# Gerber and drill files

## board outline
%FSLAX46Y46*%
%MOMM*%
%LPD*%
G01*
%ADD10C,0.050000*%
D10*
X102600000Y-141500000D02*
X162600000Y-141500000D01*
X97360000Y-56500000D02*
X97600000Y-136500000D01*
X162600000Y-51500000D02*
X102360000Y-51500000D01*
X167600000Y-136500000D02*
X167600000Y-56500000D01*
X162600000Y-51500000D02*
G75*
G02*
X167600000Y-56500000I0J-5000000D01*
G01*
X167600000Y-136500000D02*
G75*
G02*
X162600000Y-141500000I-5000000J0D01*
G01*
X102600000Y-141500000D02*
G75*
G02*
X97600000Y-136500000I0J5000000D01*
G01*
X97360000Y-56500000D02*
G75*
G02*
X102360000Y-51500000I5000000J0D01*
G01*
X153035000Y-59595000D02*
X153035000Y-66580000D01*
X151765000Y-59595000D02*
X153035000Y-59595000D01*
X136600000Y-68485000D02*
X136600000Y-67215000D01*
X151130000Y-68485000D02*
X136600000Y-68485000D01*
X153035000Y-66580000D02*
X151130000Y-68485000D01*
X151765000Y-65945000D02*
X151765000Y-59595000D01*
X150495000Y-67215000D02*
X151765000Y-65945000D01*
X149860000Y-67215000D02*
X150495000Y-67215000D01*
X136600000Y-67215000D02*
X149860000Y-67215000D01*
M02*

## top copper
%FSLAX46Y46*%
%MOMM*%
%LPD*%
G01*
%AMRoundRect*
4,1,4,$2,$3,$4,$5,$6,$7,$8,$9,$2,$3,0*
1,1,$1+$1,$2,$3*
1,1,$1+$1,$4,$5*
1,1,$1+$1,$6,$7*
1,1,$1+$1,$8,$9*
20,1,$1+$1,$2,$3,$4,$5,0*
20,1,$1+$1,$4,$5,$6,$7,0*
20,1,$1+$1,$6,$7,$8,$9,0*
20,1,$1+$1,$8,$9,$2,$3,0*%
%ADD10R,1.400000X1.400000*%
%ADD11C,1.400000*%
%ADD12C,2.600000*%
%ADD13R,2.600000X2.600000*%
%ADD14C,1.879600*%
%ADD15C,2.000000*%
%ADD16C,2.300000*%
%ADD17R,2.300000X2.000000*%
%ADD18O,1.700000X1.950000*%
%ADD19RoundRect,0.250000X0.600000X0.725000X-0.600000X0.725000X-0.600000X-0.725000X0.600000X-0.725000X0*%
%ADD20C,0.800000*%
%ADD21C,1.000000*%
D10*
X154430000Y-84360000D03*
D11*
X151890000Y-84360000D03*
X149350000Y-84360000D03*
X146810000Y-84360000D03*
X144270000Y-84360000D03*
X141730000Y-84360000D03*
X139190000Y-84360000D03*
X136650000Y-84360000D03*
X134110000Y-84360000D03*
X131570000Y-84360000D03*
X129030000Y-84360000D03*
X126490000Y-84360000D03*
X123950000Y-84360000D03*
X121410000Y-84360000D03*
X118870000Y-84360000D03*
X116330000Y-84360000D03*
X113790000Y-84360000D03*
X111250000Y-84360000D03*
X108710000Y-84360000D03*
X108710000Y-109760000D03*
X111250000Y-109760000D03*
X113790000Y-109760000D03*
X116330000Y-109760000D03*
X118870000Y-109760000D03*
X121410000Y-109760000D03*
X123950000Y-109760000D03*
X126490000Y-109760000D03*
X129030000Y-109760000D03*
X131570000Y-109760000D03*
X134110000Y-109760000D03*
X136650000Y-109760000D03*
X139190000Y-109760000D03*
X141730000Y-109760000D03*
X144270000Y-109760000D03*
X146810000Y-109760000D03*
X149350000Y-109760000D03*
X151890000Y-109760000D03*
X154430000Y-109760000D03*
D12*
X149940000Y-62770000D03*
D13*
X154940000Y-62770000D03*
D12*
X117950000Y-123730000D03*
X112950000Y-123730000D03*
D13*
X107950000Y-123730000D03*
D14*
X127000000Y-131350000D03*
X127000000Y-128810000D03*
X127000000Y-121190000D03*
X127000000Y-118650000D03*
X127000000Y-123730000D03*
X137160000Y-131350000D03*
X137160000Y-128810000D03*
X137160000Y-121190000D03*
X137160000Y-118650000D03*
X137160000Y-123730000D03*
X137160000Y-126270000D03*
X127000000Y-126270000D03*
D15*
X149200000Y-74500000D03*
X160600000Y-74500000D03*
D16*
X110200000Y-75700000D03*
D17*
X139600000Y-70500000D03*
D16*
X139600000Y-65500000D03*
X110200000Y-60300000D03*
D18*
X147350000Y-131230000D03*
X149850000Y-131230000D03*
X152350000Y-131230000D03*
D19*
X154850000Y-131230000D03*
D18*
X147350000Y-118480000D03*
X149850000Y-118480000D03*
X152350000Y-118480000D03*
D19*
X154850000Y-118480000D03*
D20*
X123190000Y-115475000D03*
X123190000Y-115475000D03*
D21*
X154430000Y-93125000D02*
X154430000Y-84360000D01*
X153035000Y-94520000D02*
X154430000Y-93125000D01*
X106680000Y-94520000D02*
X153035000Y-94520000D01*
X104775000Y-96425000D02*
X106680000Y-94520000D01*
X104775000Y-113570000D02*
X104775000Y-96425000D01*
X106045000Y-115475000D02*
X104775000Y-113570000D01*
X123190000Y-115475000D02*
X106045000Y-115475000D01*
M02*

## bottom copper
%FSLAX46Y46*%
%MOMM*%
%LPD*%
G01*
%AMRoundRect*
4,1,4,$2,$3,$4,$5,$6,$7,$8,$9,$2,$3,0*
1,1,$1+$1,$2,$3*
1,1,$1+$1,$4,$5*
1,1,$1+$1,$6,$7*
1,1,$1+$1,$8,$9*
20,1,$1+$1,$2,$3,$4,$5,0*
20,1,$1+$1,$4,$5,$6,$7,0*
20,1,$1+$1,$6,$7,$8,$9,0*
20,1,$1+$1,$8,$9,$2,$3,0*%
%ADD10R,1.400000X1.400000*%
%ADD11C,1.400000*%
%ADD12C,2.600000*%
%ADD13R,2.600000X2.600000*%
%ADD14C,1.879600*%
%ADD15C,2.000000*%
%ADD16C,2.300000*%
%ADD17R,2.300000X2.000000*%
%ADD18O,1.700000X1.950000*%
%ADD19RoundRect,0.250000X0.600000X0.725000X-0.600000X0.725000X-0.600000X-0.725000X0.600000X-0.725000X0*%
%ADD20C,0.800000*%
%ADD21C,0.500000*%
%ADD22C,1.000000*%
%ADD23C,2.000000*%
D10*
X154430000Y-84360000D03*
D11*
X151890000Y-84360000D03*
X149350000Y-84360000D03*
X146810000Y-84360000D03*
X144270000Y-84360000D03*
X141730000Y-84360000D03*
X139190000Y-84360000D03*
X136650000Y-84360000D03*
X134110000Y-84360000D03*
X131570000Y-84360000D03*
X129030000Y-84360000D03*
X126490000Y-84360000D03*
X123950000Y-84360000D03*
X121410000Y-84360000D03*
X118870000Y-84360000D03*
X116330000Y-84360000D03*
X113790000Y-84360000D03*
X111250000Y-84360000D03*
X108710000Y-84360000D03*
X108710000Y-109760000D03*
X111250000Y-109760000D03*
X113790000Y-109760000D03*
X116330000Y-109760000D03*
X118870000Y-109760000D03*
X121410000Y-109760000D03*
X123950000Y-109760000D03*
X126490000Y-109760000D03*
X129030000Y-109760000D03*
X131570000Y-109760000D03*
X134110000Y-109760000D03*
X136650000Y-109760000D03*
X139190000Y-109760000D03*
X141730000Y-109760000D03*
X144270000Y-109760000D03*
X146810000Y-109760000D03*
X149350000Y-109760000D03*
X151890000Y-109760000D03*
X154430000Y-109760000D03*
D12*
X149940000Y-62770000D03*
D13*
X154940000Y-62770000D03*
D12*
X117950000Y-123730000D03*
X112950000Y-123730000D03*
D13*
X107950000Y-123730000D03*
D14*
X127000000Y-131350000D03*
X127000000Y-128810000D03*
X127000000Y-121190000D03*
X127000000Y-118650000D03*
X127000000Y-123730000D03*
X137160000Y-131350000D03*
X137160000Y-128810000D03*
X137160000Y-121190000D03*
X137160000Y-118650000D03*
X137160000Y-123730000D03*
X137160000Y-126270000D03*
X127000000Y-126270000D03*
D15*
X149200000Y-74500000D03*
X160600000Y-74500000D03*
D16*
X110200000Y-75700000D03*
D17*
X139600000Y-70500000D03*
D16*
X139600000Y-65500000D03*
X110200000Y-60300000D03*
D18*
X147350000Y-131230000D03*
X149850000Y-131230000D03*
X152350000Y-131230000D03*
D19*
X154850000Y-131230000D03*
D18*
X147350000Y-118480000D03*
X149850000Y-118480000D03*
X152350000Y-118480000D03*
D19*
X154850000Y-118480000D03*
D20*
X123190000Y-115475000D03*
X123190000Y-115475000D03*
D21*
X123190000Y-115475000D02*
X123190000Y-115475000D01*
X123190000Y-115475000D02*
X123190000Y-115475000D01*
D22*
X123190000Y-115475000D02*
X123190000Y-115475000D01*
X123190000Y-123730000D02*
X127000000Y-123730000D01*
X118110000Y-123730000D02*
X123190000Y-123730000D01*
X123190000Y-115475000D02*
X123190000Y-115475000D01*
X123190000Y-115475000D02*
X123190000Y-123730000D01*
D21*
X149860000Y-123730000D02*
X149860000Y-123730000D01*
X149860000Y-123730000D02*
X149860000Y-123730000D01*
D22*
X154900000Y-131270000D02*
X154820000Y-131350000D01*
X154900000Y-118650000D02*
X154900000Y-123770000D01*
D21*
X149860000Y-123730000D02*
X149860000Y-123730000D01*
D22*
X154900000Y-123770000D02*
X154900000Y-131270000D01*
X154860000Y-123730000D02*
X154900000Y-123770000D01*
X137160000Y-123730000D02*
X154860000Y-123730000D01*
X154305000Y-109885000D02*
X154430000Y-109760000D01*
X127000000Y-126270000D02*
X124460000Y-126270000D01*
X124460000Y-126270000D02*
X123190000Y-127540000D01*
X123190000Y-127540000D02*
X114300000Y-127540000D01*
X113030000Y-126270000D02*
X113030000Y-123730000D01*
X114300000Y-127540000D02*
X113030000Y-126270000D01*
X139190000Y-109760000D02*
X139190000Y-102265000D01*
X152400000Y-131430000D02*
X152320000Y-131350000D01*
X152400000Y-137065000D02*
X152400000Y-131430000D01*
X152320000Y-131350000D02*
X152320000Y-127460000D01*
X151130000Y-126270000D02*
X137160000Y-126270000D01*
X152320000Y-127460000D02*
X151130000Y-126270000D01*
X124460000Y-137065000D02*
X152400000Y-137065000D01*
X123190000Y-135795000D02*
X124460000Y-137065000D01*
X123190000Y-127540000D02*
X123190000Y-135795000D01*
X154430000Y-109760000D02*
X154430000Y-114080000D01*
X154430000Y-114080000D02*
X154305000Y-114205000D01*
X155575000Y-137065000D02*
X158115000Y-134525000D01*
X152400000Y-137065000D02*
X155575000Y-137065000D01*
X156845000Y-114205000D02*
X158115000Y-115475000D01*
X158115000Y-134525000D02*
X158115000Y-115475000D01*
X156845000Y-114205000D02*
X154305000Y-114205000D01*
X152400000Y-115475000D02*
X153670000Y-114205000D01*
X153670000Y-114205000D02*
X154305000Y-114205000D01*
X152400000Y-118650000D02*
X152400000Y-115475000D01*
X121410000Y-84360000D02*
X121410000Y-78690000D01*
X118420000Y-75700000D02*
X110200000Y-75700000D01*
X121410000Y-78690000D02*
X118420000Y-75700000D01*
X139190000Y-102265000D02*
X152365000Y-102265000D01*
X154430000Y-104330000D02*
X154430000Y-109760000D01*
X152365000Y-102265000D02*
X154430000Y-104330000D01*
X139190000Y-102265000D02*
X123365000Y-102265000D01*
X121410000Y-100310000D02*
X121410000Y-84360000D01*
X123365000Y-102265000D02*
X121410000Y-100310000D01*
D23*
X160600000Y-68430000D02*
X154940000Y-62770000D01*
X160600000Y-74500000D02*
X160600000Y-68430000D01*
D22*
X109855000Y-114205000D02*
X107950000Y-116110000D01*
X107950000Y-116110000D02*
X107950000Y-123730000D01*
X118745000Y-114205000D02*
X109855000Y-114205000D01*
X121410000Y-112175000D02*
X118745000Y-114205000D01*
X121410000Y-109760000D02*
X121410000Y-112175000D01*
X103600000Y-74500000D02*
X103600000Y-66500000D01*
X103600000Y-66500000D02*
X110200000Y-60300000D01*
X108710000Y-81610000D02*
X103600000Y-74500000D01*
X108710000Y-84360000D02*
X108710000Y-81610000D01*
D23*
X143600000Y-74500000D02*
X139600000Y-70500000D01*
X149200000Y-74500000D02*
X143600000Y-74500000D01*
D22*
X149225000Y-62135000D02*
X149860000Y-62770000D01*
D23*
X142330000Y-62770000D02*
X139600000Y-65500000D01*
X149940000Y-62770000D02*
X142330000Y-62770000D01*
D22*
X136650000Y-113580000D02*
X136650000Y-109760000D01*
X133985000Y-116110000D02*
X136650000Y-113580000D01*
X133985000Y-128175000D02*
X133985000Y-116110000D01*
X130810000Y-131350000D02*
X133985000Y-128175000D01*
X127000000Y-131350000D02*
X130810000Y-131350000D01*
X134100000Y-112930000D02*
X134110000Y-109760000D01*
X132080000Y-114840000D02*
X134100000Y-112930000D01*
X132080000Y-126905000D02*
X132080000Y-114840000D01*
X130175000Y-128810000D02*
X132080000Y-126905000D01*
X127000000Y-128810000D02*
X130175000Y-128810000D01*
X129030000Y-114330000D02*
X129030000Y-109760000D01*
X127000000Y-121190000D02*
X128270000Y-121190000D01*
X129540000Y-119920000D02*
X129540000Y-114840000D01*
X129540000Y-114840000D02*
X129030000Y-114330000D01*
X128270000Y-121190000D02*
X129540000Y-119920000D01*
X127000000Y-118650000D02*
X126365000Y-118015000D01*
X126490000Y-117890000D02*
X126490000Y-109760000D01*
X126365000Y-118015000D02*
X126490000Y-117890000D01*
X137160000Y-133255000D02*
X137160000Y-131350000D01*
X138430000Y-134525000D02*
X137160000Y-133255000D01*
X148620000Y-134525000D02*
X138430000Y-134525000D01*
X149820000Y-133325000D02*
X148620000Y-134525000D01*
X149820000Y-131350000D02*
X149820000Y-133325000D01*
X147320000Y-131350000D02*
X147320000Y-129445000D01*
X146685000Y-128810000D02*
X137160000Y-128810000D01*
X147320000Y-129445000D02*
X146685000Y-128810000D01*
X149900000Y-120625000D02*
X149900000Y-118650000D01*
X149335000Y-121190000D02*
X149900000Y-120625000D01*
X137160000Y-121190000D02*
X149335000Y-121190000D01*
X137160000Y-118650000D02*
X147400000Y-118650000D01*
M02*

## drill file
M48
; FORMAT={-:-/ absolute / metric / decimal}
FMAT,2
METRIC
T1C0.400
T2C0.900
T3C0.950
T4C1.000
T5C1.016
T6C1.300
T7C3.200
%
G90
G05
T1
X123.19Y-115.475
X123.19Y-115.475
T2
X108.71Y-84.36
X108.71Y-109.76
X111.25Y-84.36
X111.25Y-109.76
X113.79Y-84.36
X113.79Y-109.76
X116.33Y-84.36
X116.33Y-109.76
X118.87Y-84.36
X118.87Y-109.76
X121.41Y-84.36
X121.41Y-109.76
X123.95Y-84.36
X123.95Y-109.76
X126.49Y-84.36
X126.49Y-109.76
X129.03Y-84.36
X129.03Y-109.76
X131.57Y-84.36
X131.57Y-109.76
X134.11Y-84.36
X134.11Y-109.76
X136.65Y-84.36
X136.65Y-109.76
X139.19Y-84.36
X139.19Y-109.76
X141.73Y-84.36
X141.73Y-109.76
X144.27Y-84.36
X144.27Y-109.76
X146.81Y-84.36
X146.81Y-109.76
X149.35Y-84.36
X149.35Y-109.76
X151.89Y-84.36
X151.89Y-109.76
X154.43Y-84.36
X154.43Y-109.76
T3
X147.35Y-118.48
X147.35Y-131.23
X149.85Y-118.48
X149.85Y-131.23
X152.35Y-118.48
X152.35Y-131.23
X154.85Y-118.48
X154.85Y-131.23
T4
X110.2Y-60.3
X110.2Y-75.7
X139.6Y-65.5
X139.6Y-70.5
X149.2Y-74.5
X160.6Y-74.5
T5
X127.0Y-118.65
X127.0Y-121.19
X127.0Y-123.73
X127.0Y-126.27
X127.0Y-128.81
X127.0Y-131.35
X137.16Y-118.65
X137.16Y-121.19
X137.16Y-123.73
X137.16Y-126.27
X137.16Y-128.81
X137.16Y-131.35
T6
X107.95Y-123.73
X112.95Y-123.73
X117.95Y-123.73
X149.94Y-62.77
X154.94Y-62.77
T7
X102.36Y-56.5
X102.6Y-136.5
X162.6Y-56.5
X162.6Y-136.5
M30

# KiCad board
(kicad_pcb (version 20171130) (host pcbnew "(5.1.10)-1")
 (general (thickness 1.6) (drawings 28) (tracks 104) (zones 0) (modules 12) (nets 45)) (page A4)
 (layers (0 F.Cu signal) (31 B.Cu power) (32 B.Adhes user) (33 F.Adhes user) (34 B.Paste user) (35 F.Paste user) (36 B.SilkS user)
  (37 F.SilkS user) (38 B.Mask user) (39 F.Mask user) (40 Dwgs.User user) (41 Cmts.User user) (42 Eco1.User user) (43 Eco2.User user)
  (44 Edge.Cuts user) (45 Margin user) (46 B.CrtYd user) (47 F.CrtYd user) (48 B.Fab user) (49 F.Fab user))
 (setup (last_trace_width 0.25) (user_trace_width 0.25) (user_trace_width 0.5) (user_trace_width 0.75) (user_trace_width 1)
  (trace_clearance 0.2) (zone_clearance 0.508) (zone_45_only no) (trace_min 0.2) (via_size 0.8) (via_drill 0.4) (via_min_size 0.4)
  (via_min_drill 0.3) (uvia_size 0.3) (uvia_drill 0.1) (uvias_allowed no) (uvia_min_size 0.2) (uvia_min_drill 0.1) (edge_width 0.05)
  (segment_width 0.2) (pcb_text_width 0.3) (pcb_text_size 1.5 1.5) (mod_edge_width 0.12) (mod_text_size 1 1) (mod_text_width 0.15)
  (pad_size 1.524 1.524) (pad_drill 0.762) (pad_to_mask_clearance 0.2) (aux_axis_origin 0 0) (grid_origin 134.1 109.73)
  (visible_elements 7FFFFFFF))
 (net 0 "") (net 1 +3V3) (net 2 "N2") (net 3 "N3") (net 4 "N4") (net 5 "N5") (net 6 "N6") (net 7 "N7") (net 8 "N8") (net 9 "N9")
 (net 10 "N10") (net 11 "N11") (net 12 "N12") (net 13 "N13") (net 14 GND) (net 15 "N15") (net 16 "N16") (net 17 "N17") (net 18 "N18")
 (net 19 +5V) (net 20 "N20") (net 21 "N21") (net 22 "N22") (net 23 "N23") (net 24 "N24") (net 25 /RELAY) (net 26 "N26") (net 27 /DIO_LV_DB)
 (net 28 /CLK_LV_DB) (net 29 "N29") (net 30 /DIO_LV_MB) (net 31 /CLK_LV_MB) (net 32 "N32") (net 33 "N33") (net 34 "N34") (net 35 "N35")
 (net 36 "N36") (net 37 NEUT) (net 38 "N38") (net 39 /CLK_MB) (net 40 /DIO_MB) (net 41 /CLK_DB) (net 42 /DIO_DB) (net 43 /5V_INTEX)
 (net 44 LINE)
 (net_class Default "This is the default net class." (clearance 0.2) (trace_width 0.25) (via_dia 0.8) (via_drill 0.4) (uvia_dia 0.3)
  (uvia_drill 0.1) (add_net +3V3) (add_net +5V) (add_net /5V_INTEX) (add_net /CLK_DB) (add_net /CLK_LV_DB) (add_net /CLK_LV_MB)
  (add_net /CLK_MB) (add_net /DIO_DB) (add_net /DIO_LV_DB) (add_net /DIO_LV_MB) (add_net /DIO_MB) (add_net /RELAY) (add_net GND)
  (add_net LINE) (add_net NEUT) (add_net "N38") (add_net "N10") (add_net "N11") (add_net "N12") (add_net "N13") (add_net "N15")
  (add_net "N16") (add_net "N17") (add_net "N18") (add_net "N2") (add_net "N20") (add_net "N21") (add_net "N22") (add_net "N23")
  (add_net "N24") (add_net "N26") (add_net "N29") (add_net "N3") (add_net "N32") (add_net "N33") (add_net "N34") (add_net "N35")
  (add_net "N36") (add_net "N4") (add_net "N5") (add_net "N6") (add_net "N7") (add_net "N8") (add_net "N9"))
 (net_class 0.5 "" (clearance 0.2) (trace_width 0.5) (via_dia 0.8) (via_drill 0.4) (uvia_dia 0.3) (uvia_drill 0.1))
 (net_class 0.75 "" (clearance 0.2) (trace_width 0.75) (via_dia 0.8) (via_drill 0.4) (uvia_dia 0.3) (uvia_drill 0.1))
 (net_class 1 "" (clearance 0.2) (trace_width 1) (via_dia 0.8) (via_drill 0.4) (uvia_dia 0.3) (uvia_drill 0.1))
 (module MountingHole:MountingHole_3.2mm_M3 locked (layer F.Cu) (at 162.6 136.5)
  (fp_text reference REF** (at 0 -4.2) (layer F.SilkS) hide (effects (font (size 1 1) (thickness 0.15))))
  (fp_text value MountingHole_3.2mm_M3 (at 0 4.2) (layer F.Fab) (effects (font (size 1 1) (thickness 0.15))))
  (pad 1 np_thru_hole circle (at 0 0) (size 3.2 3.2) (drill 3.2) (layers *.Cu *.Mask)))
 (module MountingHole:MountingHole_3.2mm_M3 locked (layer F.Cu) (at 102.6 136.5)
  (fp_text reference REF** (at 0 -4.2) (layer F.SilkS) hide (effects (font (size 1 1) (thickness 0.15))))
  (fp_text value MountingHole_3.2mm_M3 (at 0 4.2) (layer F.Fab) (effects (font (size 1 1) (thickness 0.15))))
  (pad 1 np_thru_hole circle (at 0 0) (size 3.2 3.2) (drill 3.2) (layers *.Cu *.Mask)))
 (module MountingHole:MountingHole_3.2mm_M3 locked (layer F.Cu) (at 162.6 56.5)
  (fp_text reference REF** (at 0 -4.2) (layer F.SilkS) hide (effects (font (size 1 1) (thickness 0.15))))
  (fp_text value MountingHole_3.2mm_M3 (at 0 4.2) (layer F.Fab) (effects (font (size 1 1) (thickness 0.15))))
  (pad 1 np_thru_hole circle (at 0 0) (size 3.2 3.2) (drill 3.2) (layers *.Cu *.Mask)))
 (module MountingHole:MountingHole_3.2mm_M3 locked (layer F.Cu) (at 102.36 56.5)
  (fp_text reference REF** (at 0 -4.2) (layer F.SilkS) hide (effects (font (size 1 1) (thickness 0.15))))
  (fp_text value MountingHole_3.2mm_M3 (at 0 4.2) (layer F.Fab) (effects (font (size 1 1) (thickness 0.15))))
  (pad 1 np_thru_hole circle (at 0 0) (size 3.2 3.2) (drill 3.2) (layers *.Cu *.Mask)))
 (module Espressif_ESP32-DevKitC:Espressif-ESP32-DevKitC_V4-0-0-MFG (layer F.Cu) (at 134.62 97.06 270)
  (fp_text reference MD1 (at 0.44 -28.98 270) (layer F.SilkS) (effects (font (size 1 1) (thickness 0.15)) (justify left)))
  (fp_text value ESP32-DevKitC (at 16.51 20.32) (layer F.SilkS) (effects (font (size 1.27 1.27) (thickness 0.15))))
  (pad 1 thru_hole rect (at -12.7 -19.81 270) (size 1.4 1.4) (drill 0.9) (layers *.Cu *.Paste *.Mask) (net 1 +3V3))
  (pad 2 thru_hole circle (at -12.7 -17.27 270) (size 1.4 1.4) (drill 0.9) (layers *.Cu *.Paste *.Mask) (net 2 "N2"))
  (pad 3 thru_hole circle (at -12.7 -14.73 270) (size 1.4 1.4) (drill 0.9) (layers *.Cu *.Paste *.Mask) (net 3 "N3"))
  (pad 4 thru_hole circle (at -12.7 -12.19 270) (size 1.4 1.4) (drill 0.9) (layers *.Cu *.Paste *.Mask) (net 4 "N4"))
  (pad 5 thru_hole circle (at -12.7 -9.65 270) (size 1.4 1.4) (drill 0.9) (layers *.Cu *.Paste *.Mask) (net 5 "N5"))
  (pad 6 thru_hole circle (at -12.7 -7.11 270) (size 1.4 1.4) (drill 0.9) (layers *.Cu *.Paste *.Mask) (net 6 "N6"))
  (pad 7 thru_hole circle (at -12.7 -4.57 270) (size 1.4 1.4) (drill 0.9) (layers *.Cu *.Paste *.Mask) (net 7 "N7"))
  (pad 8 thru_hole circle (at -12.7 -2.03 270) (size 1.4 1.4) (drill 0.9) (layers *.Cu *.Paste *.Mask) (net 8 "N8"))
  (pad 9 thru_hole circle (at -12.7 0.51 270) (size 1.4 1.4) (drill 0.9) (layers *.Cu *.Paste *.Mask) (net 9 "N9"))
  (pad 10 thru_hole circle (at -12.7 3.05 270) (size 1.4 1.4) (drill 0.9) (layers *.Cu *.Paste *.Mask) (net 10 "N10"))
  (pad 11 thru_hole circle (at -12.7 5.59 270) (size 1.4 1.4) (drill 0.9) (layers *.Cu *.Paste *.Mask) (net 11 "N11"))
  (pad 12 thru_hole circle (at -12.7 8.13 270) (size 1.4 1.4) (drill 0.9) (layers *.Cu *.Paste *.Mask) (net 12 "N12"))
  (pad 13 thru_hole circle (at -12.7 10.67 270) (size 1.4 1.4) (drill 0.9) (layers *.Cu *.Paste *.Mask) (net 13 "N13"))
  (pad 14 thru_hole circle (at -12.7 13.21 270) (size 1.4 1.4) (drill 0.9) (layers *.Cu *.Paste *.Mask) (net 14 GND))
  (pad 15 thru_hole circle (at -12.7 15.75 270) (size 1.4 1.4) (drill 0.9) (layers *.Cu *.Paste *.Mask) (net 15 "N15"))
  (pad 16 thru_hole circle (at -12.7 18.29 270) (size 1.4 1.4) (drill 0.9) (layers *.Cu *.Paste *.Mask) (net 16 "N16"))
  (pad 17 thru_hole circle (at -12.7 20.83 270) (size 1.4 1.4) (drill 0.9) (layers *.Cu *.Paste *.Mask) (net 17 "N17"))
  (pad 18 thru_hole circle (at -12.7 23.37 270) (size 1.4 1.4) (drill 0.9) (layers *.Cu *.Paste *.Mask) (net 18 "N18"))
  (pad 19 thru_hole circle (at -12.7 25.91 270) (size 1.4 1.4) (drill 0.9) (layers *.Cu *.Paste *.Mask) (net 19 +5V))
  (pad 20 thru_hole circle (at 12.7 25.91 270) (size 1.4 1.4) (drill 0.9) (layers *.Cu *.Paste *.Mask) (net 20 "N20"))
  (pad 21 thru_hole circle (at 12.7 23.37 270) (size 1.4 1.4) (drill 0.9) (layers *.Cu *.Paste *.Mask) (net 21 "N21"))
  (pad 22 thru_hole circle (at 12.7 20.83 270) (size 1.4 1.4) (drill 0.9) (layers *.Cu *.Paste *.Mask) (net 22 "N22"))
  (pad 23 thru_hole circle (at 12.7 18.29 270) (size 1.4 1.4) (drill 0.9) (layers *.Cu *.Paste *.Mask) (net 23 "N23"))
  (pad 24 thru_hole circle (at 12.7 15.75 270) (size 1.4 1.4) (drill 0.9) (layers *.Cu *.Paste *.Mask) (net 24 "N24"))
  (pad 25 thru_hole circle (at 12.7 13.21 270) (size 1.4 1.4) (drill 0.9) (layers *.Cu *.Paste *.Mask) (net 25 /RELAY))
  (pad 26 thru_hole circle (at 12.7 10.67 270) (size 1.4 1.4) (drill 0.9) (layers *.Cu *.Paste *.Mask) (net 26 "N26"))
  (pad 27 thru_hole circle (at 12.7 8.13 270) (size 1.4 1.4) (drill 0.9) (layers *.Cu *.Paste *.Mask) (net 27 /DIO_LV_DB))
  (pad 28 thru_hole circle (at 12.7 5.59 270) (size 1.4 1.4) (drill 0.9) (layers *.Cu *.Paste *.Mask) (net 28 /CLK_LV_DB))
  (pad 29 thru_hole circle (at 12.7 3.05 270) (size 1.4 1.4) (drill 0.9) (layers *.Cu *.Paste *.Mask) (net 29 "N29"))
  (pad 30 thru_hole circle (at 12.7 0.51 270) (size 1.4 1.4) (drill 0.9) (layers *.Cu *.Paste *.Mask) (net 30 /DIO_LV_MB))
  (pad 31 thru_hole circle (at 12.7 -2.03 270) (size 1.4 1.4) (drill 0.9) (layers *.Cu *.Paste *.Mask) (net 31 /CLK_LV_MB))
  (pad 32 thru_hole circle (at 12.7 -4.57 270) (size 1.4 1.4) (drill 0.9) (layers *.Cu *.Paste *.Mask) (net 14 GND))
  (pad 33 thru_hole circle (at 12.7 -7.11 270) (size 1.4 1.4) (drill 0.9) (layers *.Cu *.Paste *.Mask) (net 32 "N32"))
  (pad 34 thru_hole circle (at 12.7 -9.65 270) (size 1.4 1.4) (drill 0.9) (layers *.Cu *.Paste *.Mask) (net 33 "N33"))
  (pad 35 thru_hole circle (at 12.7 -12.19 270) (size 1.4 1.4) (drill 0.9) (layers *.Cu *.Paste *.Mask) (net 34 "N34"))
  (pad 36 thru_hole circle (at 12.7 -14.73 270) (size 1.4 1.4) (drill 0.9) (layers *.Cu *.Paste *.Mask) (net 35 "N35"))
  (pad 37 thru_hole circle (at 12.7 -17.27 270) (size 1.4 1.4) (drill 0.9) (layers *.Cu *.Paste *.Mask) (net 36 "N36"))
  (pad 38 thru_hole circle (at 12.7 -19.81 270) (size 1.4 1.4) (drill 0.9) (layers *.Cu *.Paste *.Mask) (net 14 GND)))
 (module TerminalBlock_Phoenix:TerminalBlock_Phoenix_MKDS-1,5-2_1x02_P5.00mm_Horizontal (layer F.Cu) (at 154.94 62.77 180)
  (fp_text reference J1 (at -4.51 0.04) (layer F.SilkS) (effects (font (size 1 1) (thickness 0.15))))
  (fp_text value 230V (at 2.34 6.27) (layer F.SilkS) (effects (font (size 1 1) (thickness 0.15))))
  (pad 2 thru_hole circle (at 5 0 180) (size 2.6 2.6) (drill 1.3) (layers *.Cu *.Mask) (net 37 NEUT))
  (pad 1 thru_hole rect (at 0 0 180) (size 2.6 2.6) (drill 1.3) (layers *.Cu *.Mask) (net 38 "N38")))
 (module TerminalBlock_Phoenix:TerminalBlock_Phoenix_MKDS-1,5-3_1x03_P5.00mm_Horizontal (layer F.Cu) (at 107.95 123.73)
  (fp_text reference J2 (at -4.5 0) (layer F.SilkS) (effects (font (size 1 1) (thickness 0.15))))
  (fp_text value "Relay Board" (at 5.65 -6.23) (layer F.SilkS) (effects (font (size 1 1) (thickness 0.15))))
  (pad 3 thru_hole circle (at 10 0) (size 2.6 2.6) (drill 1.3) (layers *.Cu *.Mask) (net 1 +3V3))
  (pad 2 thru_hole circle (at 5 0) (size 2.6 2.6) (drill 1.3) (layers *.Cu *.Mask) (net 14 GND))
  (pad 1 thru_hole rect (at 0 0) (size 2.6 2.6) (drill 1.3) (layers *.Cu *.Mask) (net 25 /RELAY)))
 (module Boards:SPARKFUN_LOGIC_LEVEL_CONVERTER (layer F.Cu) (at 132.08 125)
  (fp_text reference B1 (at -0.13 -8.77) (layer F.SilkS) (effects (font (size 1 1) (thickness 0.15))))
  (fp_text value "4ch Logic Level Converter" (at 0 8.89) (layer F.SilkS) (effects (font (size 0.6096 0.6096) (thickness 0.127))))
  (pad LV4 thru_hole circle (at -5.08 6.35) (size 1.8796 1.8796) (drill 1.016) (layers *.Cu *.Mask) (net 31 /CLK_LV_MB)
   (solder_mask_margin 0.1016))
  (pad LV3 thru_hole circle (at -5.08 3.81) (size 1.8796 1.8796) (drill 1.016) (layers *.Cu *.Mask) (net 30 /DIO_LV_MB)
   (solder_mask_margin 0.1016))
  (pad LV2 thru_hole circle (at -5.08 -3.81) (size 1.8796 1.8796) (drill 1.016) (layers *.Cu *.Mask) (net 28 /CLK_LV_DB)
   (solder_mask_margin 0.1016))
  (pad LV1 thru_hole circle (at -5.08 -6.35) (size 1.8796 1.8796) (drill 1.016) (layers *.Cu *.Mask) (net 27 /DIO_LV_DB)
   (solder_mask_margin 0.1016))
  (pad LV thru_hole circle (at -5.08 -1.27) (size 1.8796 1.8796) (drill 1.016) (layers *.Cu *.Mask) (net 1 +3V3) (solder_mask_margin 0.1016))
  (pad HV4 thru_hole circle (at 5.08 6.35) (size 1.8796 1.8796) (drill 1.016) (layers *.Cu *.Mask) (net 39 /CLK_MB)
   (solder_mask_margin 0.1016))
  (pad HV3 thru_hole circle (at 5.08 3.81) (size 1.8796 1.8796) (drill 1.016) (layers *.Cu *.Mask) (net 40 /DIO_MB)
   (solder_mask_margin 0.1016))
  (pad HV2 thru_hole circle (at 5.08 -3.81) (size 1.8796 1.8796) (drill 1.016) (layers *.Cu *.Mask) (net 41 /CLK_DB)
   (solder_mask_margin 0.1016))
  (pad HV1 thru_hole circle (at 5.08 -6.35) (size 1.8796 1.8796) (drill 1.016) (layers *.Cu *.Mask) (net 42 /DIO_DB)
   (solder_mask_margin 0.1016))
  (pad HV thru_hole circle (at 5.08 -1.27) (size 1.8796 1.8796) (drill 1.016) (layers *.Cu *.Mask) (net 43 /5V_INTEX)
   (solder_mask_margin 0.1016))
  (pad GND2 thru_hole circle (at 5.08 1.27) (size 1.8796 1.8796) (drill 1.016) (layers *.Cu *.Mask) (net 14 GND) (solder_mask_margin 0.1016))
  (pad GND1 thru_hole circle (at -5.08 1.27) (size 1.8796 1.8796) (drill 1.016) (layers *.Cu *.Mask) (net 14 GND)
   (solder_mask_margin 0.1016)))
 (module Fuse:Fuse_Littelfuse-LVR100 (layer F.Cu) (at 160.6 74.5 180)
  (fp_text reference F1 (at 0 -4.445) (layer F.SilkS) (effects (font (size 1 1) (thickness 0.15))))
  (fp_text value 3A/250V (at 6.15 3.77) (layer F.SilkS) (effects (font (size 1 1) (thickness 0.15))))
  (pad 2 thru_hole circle (at 11.4 0 180) (size 2 2) (drill 1) (layers *.Cu *.Mask) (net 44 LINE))
  (pad 1 thru_hole circle (at 0 0 180) (size 2 2) (drill 1) (layers *.Cu *.Mask) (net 38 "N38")))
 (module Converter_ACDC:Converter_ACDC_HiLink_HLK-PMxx (layer F.Cu) (at 139.6 70.5 180)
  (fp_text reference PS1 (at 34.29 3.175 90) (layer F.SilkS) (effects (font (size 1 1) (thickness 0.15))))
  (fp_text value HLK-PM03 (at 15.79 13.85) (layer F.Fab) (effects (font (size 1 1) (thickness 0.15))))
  (pad 3 thru_hole circle (at 29.4 -5.2 180) (size 2.3 2.3) (drill 1) (layers *.Cu *.Mask) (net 14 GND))
  (pad 1 thru_hole rect (at 0 0 180) (size 2.3 2) (drill 1) (layers *.Cu *.Mask) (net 44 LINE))
  (pad 2 thru_hole circle (at 0 5 180) (size 2.3 2.3) (drill 1) (layers *.Cu *.Mask) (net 37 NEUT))
  (pad 4 thru_hole circle (at 29.4 10.2 180) (size 2.3 2.3) (drill 1) (layers *.Cu *.Mask) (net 19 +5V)))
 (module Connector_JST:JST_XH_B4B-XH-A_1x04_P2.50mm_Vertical (layer F.Cu) (at 154.85 131.23 180)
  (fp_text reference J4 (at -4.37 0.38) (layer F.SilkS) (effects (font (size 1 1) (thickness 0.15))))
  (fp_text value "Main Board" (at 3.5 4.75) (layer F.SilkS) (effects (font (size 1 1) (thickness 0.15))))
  (pad 4 thru_hole oval (at 7.5 0 180) (size 1.7 1.95) (drill 0.95) (layers *.Cu *.Mask) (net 40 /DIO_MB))
  (pad 3 thru_hole oval (at 5 0 180) (size 1.7 1.95) (drill 0.95) (layers *.Cu *.Mask) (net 39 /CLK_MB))
  (pad 2 thru_hole oval (at 2.5 0 180) (size 1.7 1.95) (drill 0.95) (layers *.Cu *.Mask) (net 14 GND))
  (pad 1 thru_hole roundrect (at 0 0 180) (size 1.7 1.95) (drill 0.95) (layers *.Cu *.Mask) (roundrect_rratio 0.1470588235294118)
   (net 43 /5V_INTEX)))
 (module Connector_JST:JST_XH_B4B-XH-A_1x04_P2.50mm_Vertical (layer F.Cu) (at 154.85 118.48 180)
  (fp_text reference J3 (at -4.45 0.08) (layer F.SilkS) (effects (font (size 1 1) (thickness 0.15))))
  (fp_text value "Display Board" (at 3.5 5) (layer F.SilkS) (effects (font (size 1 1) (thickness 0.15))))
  (pad 4 thru_hole oval (at 7.5 0 180) (size 1.7 1.95) (drill 0.95) (layers *.Cu *.Mask) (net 42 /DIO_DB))
  (pad 3 thru_hole oval (at 5 0 180) (size 1.7 1.95) (drill 0.95) (layers *.Cu *.Mask) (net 41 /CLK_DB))
  (pad 2 thru_hole oval (at 2.5 0 180) (size 1.7 1.95) (drill 0.95) (layers *.Cu *.Mask) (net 14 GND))
  (pad 1 thru_hole roundrect (at 0 0 180) (size 1.7 1.95) (drill 0.95) (layers *.Cu *.Mask) (roundrect_rratio 0.1470588235294118)
   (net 43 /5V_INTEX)))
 (gr_line (start 102.6 141.5) (end 162.6 141.5) (layer Edge.Cuts) (width 0.05))
 (gr_line (start 97.36 56.5) (end 97.6 136.5) (layer Edge.Cuts) (width 0.05))
 (gr_line (start 162.6 51.5) (end 102.36 51.5) (layer Edge.Cuts) (width 0.05))
 (gr_line (start 167.6 136.5) (end 167.6 56.5) (layer Edge.Cuts) (width 0.05))
 (gr_arc (start 162.6 56.5) (end 167.6 56.5) (angle -90) (layer Edge.Cuts) (width 0.05))
 (gr_arc (start 162.6 136.5) (end 162.6 141.5) (angle -90) (layer Edge.Cuts) (width 0.05))
 (gr_arc (start 102.6 136.5) (end 97.6 136.5) (angle -90) (layer Edge.Cuts) (width 0.05))
 (gr_arc (start 102.36 56.5) (end 102.36 51.5) (angle -90) (layer Edge.Cuts) (width 0.05))
 (gr_line (start 153.035 59.595) (end 153.035 66.58) (layer Edge.Cuts) (width 0.05))
 (gr_line (start 151.765 59.595) (end 153.035 59.595) (layer Edge.Cuts) (width 0.05))
 (gr_line (start 136.6 68.485) (end 136.6 67.215) (layer Edge.Cuts) (width 0.05))
 (gr_line (start 151.13 68.485) (end 136.6 68.485) (layer Edge.Cuts) (width 0.05))
 (gr_line (start 153.035 66.58) (end 151.13 68.485) (layer Edge.Cuts) (width 0.05))
 (gr_line (start 151.765 65.945) (end 151.765 59.595) (layer Edge.Cuts) (width 0.05))
 (gr_line (start 150.495 67.215) (end 151.765 65.945) (layer Edge.Cuts) (width 0.05))
 (gr_line (start 149.86 67.215) (end 150.495 67.215) (layer Edge.Cuts) (width 0.05))
 (gr_line (start 136.6 67.215) (end 149.86 67.215) (layer Edge.Cuts) (width 0.05))
 (segment (start 123.19 115.475) (end 123.19 115.475) (width 0.5) (layer B.Cu) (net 1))
 (segment (start 123.19 115.475) (end 123.19 115.475) (width 0.5) (layer B.Cu) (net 1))
 (segment (start 123.19 115.475) (end 123.19 115.475) (width 1) (layer B.Cu) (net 1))
 (segment (start 123.19 123.73) (end 127 123.73) (width 1) (layer B.Cu) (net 1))
 (segment (start 118.11 123.73) (end 123.19 123.73) (width 1) (layer B.Cu) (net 1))
 (segment (start 123.19 115.475) (end 123.19 115.475) (width 1) (layer B.Cu) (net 1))
 (via (at 123.19 115.475) (size 0.8) (drill 0.4) (layers F.Cu B.Cu) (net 1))
 (segment (start 123.19 115.475) (end 123.19 123.73) (width 1) (layer B.Cu) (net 1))
 (via (at 123.19 115.475) (size 0.8) (drill 0.4) (layers F.Cu B.Cu) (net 1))
 (segment (start 154.43 93.125) (end 154.43 84.36) (width 1) (layer F.Cu) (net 1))
 (segment (start 153.035 94.52) (end 154.43 93.125) (width 1) (layer F.Cu) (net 1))
 (segment (start 106.68 94.52) (end 153.035 94.52) (width 1) (layer F.Cu) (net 1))
 (segment (start 104.775 96.425) (end 106.68 94.52) (width 1) (layer F.Cu) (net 1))
 (segment (start 104.775 113.57) (end 104.775 96.425) (width 1) (layer F.Cu) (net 1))
 (segment (start 106.045 115.475) (end 104.775 113.57) (width 1) (layer F.Cu) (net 1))
 (segment (start 123.19 115.475) (end 106.045 115.475) (width 1) (layer F.Cu) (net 1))
 (segment (start 149.86 123.73) (end 149.86 123.73) (width 0.5) (layer B.Cu) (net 43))
 (segment (start 149.86 123.73) (end 149.86 123.73) (width 0.5) (layer B.Cu) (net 43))
 (segment (start 154.9 131.27) (end 154.82 131.35) (width 1) (layer B.Cu) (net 43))
 (segment (start 154.9 118.65) (end 154.9 123.77) (width 1) (layer B.Cu) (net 43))
 (segment (start 149.86 123.73) (end 149.86 123.73) (width 0.5) (layer B.Cu) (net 43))
 (segment (start 154.9 123.77) (end 154.9 131.27) (width 1) (layer B.Cu) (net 43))
 (segment (start 154.86 123.73) (end 154.9 123.77) (width 1) (layer B.Cu) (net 43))
 (segment (start 137.16 123.73) (end 154.86 123.73) (width 1) (layer B.Cu) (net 43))
 (segment (start 154.305 109.885) (end 154.43 109.76) (width 1) (layer B.Cu) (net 14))
 (segment (start 127 126.27) (end 124.46 126.27) (width 1) (layer B.Cu) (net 14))
 (segment (start 124.46 126.27) (end 123.19 127.54) (width 1) (layer B.Cu) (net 14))
 (segment (start 123.19 127.54) (end 114.3 127.54) (width 1) (layer B.Cu) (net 14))
 (segment (start 113.03 126.27) (end 113.03 123.73) (width 1) (layer B.Cu) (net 14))
 (segment (start 114.3 127.54) (end 113.03 126.27) (width 1) (layer B.Cu) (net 14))
 (segment (start 139.19 109.76) (end 139.19 102.265) (width 1) (layer B.Cu) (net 14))
 (segment (start 152.4 131.43) (end 152.32 131.35) (width 1) (layer B.Cu) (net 14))
 (segment (start 152.4 137.065) (end 152.4 131.43) (width 1) (layer B.Cu) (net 14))
 (segment (start 152.32 131.35) (end 152.32 127.46) (width 1) (layer B.Cu) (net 14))
 (segment (start 151.13 126.27) (end 137.16 126.27) (width 1) (layer B.Cu) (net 14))
 (segment (start 152.32 127.46) (end 151.13 126.27) (width 1) (layer B.Cu) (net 14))
 (segment (start 124.46 137.065) (end 152.4 137.065) (width 1) (layer B.Cu) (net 14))
 (segment (start 123.19 135.795) (end 124.46 137.065) (width 1) (layer B.Cu) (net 14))
 (segment (start 123.19 127.54) (end 123.19 135.795) (width 1) (layer B.Cu) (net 14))
 (segment (start 154.43 109.76) (end 154.43 114.08) (width 1) (layer B.Cu) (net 14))
 (segment (start 154.43 114.08) (end 154.305 114.205) (width 1) (layer B.Cu) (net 14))
 (segment (start 155.575 137.065) (end 158.115 134.525) (width 1) (layer B.Cu) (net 14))
 (segment (start 152.4 137.065) (end 155.575 137.065) (width 1) (layer B.Cu) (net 14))
 (segment (start 156.845 114.205) (end 158.115 115.475) (width 1) (layer B.Cu) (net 14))
 (segment (start 158.115 134.525) (end 158.115 115.475) (width 1) (layer B.Cu) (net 14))
 (segment (start 156.845 114.205) (end 154.305 114.205) (width 1) (layer B.Cu) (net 14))
 (segment (start 152.4 115.475) (end 153.67 114.205) (width 1) (layer B.Cu) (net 14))
 (segment (start 153.67 114.205) (end 154.305 114.205) (width 1) (layer B.Cu) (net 14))
 (segment (start 152.4 118.65) (end 152.4 115.475) (width 1) (layer B.Cu) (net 14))
 (segment (start 121.41 84.36) (end 121.41 78.69) (width 1) (layer B.Cu) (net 14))
 (segment (start 118.42 75.7) (end 110.2 75.7) (width 1) (layer B.Cu) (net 14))
 (segment (start 121.41 78.69) (end 118.42 75.7) (width 1) (layer B.Cu) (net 14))
 (segment (start 139.19 102.265) (end 152.365 102.265) (width 1) (layer B.Cu) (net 14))
 (segment (start 154.43 104.33) (end 154.43 109.76) (width 1) (layer B.Cu) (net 14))
 (segment (start 152.365 102.265) (end 154.43 104.33) (width 1) (layer B.Cu) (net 14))
 (segment (start 139.19 102.265) (end 123.365 102.265) (width 1) (layer B.Cu) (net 14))
 (segment (start 121.41 100.31) (end 121.41 84.36) (width 1) (layer B.Cu) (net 14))
 (segment (start 123.365 102.265) (end 121.41 100.31) (width 1) (layer B.Cu) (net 14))
 (segment (start 160.6 68.43) (end 154.94 62.77) (width 2) (layer B.Cu) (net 38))
 (segment (start 160.6 74.5) (end 160.6 68.43) (width 2) (layer B.Cu) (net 38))
 (segment (start 109.855 114.205) (end 107.95 116.11) (width 1) (layer B.Cu) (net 25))
 (segment (start 107.95 116.11) (end 107.95 123.73) (width 1) (layer B.Cu) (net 25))
 (segment (start 118.745 114.205) (end 109.855 114.205) (width 1) (layer B.Cu) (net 25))
 (segment (start 121.41 112.175) (end 118.745 114.205) (width 1) (layer B.Cu) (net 25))
 (segment (start 121.41 109.76) (end 121.41 112.175) (width 1) (layer B.Cu) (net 25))
 (segment (start 103.6 74.5) (end 103.6 66.5) (width 1) (layer B.Cu) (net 19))
 (segment (start 103.6 66.5) (end 110.2 60.3) (width 1) (layer B.Cu) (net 19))
 (segment (start 108.71 81.61) (end 103.6 74.5) (width 1) (layer B.Cu) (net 19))
 (segment (start 108.71 84.36) (end 108.71 81.61) (width 1) (layer B.Cu) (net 19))
 (segment (start 143.6 74.5) (end 139.6 70.5) (width 2) (layer B.Cu) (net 44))
 (segment (start 149.2 74.5) (end 143.6 74.5) (width 2) (layer B.Cu) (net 44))
 (segment (start 149.225 62.135) (end 149.86 62.77) (width 1) (layer B.Cu) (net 37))
 (segment (start 142.33 62.77) (end 139.6 65.5) (width 2) (layer B.Cu) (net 37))
 (segment (start 149.94 62.77) (end 142.33 62.77) (width 2) (layer B.Cu) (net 37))
 (segment (start 136.65 113.58) (end 136.65 109.76) (width 1) (layer B.Cu) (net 31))
 (segment (start 133.985 116.11) (end 136.65 113.58) (width 1) (layer B.Cu) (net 31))
 (segment (start 133.985 128.175) (end 133.985 116.11) (width 1) (layer B.Cu) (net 31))
 (segment (start 130.81 131.35) (end 133.985 128.175) (width 1) (layer B.Cu) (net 31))
 (segment (start 127 131.35) (end 130.81 131.35) (width 1) (layer B.Cu) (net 31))
 (segment (start 134.1 112.93) (end 134.11 109.76) (width 1) (layer B.Cu) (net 30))
 (segment (start 132.08 114.84) (end 134.1 112.93) (width 1) (layer B.Cu) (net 30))
 (segment (start 132.08 126.905) (end 132.08 114.84) (width 1) (layer B.Cu) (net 30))
 (segment (start 130.175 128.81) (end 132.08 126.905) (width 1) (layer B.Cu) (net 30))
 (segment (start 127 128.81) (end 130.175 128.81) (width 1) (layer B.Cu) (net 30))
 (segment (start 129.03 114.33) (end 129.03 109.76) (width 1) (layer B.Cu) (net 28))
 (segment (start 127 121.19) (end 128.27 121.19) (width 1) (layer B.Cu) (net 28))
 (segment (start 129.54 119.92) (end 129.54 114.84) (width 1) (layer B.Cu) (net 28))
 (segment (start 129.54 114.84) (end 129.03 114.33) (width 1) (layer B.Cu) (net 28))
 (segment (start 128.27 121.19) (end 129.54 119.92) (width 1) (layer B.Cu) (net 28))
 (segment (start 127 118.65) (end 126.365 118.015) (width 1) (layer B.Cu) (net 27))
 (segment (start 126.49 117.89) (end 126.49 109.76) (width 1) (layer B.Cu) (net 27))
 (segment (start 126.365 118.015) (end 126.49 117.89) (width 1) (layer B.Cu) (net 27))
 (segment (start 137.16 133.255) (end 137.16 131.35) (width 1) (layer B.Cu) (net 39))
 (segment (start 138.43 134.525) (end 137.16 133.255) (width 1) (layer B.Cu) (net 39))
 (segment (start 148.62 134.525) (end 138.43 134.525) (width 1) (layer B.Cu) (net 39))
 (segment (start 149.82 133.325) (end 148.62 134.525) (width 1) (layer B.Cu) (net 39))
 (segment (start 149.82 131.35) (end 149.82 133.325) (width 1) (layer B.Cu) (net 39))
 (segment (start 147.32 131.35) (end 147.32 129.445) (width 1) (layer B.Cu) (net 40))
 (segment (start 146.685 128.81) (end 137.16 128.81) (width 1) (layer B.Cu) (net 40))
 (segment (start 147.32 129.445) (end 146.685 128.81) (width 1) (layer B.Cu) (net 40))
 (segment (start 149.9 120.625) (end 149.9 118.65) (width 1) (layer B.Cu) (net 41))
 (segment (start 149.335 121.19) (end 149.9 120.625) (width 1) (layer B.Cu) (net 41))
 (segment (start 137.16 121.19) (end 149.335 121.19) (width 1) (layer B.Cu) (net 41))
 (segment (start 137.16 118.65) (end 147.4 118.65) (width 1) (layer B.Cu) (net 42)))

